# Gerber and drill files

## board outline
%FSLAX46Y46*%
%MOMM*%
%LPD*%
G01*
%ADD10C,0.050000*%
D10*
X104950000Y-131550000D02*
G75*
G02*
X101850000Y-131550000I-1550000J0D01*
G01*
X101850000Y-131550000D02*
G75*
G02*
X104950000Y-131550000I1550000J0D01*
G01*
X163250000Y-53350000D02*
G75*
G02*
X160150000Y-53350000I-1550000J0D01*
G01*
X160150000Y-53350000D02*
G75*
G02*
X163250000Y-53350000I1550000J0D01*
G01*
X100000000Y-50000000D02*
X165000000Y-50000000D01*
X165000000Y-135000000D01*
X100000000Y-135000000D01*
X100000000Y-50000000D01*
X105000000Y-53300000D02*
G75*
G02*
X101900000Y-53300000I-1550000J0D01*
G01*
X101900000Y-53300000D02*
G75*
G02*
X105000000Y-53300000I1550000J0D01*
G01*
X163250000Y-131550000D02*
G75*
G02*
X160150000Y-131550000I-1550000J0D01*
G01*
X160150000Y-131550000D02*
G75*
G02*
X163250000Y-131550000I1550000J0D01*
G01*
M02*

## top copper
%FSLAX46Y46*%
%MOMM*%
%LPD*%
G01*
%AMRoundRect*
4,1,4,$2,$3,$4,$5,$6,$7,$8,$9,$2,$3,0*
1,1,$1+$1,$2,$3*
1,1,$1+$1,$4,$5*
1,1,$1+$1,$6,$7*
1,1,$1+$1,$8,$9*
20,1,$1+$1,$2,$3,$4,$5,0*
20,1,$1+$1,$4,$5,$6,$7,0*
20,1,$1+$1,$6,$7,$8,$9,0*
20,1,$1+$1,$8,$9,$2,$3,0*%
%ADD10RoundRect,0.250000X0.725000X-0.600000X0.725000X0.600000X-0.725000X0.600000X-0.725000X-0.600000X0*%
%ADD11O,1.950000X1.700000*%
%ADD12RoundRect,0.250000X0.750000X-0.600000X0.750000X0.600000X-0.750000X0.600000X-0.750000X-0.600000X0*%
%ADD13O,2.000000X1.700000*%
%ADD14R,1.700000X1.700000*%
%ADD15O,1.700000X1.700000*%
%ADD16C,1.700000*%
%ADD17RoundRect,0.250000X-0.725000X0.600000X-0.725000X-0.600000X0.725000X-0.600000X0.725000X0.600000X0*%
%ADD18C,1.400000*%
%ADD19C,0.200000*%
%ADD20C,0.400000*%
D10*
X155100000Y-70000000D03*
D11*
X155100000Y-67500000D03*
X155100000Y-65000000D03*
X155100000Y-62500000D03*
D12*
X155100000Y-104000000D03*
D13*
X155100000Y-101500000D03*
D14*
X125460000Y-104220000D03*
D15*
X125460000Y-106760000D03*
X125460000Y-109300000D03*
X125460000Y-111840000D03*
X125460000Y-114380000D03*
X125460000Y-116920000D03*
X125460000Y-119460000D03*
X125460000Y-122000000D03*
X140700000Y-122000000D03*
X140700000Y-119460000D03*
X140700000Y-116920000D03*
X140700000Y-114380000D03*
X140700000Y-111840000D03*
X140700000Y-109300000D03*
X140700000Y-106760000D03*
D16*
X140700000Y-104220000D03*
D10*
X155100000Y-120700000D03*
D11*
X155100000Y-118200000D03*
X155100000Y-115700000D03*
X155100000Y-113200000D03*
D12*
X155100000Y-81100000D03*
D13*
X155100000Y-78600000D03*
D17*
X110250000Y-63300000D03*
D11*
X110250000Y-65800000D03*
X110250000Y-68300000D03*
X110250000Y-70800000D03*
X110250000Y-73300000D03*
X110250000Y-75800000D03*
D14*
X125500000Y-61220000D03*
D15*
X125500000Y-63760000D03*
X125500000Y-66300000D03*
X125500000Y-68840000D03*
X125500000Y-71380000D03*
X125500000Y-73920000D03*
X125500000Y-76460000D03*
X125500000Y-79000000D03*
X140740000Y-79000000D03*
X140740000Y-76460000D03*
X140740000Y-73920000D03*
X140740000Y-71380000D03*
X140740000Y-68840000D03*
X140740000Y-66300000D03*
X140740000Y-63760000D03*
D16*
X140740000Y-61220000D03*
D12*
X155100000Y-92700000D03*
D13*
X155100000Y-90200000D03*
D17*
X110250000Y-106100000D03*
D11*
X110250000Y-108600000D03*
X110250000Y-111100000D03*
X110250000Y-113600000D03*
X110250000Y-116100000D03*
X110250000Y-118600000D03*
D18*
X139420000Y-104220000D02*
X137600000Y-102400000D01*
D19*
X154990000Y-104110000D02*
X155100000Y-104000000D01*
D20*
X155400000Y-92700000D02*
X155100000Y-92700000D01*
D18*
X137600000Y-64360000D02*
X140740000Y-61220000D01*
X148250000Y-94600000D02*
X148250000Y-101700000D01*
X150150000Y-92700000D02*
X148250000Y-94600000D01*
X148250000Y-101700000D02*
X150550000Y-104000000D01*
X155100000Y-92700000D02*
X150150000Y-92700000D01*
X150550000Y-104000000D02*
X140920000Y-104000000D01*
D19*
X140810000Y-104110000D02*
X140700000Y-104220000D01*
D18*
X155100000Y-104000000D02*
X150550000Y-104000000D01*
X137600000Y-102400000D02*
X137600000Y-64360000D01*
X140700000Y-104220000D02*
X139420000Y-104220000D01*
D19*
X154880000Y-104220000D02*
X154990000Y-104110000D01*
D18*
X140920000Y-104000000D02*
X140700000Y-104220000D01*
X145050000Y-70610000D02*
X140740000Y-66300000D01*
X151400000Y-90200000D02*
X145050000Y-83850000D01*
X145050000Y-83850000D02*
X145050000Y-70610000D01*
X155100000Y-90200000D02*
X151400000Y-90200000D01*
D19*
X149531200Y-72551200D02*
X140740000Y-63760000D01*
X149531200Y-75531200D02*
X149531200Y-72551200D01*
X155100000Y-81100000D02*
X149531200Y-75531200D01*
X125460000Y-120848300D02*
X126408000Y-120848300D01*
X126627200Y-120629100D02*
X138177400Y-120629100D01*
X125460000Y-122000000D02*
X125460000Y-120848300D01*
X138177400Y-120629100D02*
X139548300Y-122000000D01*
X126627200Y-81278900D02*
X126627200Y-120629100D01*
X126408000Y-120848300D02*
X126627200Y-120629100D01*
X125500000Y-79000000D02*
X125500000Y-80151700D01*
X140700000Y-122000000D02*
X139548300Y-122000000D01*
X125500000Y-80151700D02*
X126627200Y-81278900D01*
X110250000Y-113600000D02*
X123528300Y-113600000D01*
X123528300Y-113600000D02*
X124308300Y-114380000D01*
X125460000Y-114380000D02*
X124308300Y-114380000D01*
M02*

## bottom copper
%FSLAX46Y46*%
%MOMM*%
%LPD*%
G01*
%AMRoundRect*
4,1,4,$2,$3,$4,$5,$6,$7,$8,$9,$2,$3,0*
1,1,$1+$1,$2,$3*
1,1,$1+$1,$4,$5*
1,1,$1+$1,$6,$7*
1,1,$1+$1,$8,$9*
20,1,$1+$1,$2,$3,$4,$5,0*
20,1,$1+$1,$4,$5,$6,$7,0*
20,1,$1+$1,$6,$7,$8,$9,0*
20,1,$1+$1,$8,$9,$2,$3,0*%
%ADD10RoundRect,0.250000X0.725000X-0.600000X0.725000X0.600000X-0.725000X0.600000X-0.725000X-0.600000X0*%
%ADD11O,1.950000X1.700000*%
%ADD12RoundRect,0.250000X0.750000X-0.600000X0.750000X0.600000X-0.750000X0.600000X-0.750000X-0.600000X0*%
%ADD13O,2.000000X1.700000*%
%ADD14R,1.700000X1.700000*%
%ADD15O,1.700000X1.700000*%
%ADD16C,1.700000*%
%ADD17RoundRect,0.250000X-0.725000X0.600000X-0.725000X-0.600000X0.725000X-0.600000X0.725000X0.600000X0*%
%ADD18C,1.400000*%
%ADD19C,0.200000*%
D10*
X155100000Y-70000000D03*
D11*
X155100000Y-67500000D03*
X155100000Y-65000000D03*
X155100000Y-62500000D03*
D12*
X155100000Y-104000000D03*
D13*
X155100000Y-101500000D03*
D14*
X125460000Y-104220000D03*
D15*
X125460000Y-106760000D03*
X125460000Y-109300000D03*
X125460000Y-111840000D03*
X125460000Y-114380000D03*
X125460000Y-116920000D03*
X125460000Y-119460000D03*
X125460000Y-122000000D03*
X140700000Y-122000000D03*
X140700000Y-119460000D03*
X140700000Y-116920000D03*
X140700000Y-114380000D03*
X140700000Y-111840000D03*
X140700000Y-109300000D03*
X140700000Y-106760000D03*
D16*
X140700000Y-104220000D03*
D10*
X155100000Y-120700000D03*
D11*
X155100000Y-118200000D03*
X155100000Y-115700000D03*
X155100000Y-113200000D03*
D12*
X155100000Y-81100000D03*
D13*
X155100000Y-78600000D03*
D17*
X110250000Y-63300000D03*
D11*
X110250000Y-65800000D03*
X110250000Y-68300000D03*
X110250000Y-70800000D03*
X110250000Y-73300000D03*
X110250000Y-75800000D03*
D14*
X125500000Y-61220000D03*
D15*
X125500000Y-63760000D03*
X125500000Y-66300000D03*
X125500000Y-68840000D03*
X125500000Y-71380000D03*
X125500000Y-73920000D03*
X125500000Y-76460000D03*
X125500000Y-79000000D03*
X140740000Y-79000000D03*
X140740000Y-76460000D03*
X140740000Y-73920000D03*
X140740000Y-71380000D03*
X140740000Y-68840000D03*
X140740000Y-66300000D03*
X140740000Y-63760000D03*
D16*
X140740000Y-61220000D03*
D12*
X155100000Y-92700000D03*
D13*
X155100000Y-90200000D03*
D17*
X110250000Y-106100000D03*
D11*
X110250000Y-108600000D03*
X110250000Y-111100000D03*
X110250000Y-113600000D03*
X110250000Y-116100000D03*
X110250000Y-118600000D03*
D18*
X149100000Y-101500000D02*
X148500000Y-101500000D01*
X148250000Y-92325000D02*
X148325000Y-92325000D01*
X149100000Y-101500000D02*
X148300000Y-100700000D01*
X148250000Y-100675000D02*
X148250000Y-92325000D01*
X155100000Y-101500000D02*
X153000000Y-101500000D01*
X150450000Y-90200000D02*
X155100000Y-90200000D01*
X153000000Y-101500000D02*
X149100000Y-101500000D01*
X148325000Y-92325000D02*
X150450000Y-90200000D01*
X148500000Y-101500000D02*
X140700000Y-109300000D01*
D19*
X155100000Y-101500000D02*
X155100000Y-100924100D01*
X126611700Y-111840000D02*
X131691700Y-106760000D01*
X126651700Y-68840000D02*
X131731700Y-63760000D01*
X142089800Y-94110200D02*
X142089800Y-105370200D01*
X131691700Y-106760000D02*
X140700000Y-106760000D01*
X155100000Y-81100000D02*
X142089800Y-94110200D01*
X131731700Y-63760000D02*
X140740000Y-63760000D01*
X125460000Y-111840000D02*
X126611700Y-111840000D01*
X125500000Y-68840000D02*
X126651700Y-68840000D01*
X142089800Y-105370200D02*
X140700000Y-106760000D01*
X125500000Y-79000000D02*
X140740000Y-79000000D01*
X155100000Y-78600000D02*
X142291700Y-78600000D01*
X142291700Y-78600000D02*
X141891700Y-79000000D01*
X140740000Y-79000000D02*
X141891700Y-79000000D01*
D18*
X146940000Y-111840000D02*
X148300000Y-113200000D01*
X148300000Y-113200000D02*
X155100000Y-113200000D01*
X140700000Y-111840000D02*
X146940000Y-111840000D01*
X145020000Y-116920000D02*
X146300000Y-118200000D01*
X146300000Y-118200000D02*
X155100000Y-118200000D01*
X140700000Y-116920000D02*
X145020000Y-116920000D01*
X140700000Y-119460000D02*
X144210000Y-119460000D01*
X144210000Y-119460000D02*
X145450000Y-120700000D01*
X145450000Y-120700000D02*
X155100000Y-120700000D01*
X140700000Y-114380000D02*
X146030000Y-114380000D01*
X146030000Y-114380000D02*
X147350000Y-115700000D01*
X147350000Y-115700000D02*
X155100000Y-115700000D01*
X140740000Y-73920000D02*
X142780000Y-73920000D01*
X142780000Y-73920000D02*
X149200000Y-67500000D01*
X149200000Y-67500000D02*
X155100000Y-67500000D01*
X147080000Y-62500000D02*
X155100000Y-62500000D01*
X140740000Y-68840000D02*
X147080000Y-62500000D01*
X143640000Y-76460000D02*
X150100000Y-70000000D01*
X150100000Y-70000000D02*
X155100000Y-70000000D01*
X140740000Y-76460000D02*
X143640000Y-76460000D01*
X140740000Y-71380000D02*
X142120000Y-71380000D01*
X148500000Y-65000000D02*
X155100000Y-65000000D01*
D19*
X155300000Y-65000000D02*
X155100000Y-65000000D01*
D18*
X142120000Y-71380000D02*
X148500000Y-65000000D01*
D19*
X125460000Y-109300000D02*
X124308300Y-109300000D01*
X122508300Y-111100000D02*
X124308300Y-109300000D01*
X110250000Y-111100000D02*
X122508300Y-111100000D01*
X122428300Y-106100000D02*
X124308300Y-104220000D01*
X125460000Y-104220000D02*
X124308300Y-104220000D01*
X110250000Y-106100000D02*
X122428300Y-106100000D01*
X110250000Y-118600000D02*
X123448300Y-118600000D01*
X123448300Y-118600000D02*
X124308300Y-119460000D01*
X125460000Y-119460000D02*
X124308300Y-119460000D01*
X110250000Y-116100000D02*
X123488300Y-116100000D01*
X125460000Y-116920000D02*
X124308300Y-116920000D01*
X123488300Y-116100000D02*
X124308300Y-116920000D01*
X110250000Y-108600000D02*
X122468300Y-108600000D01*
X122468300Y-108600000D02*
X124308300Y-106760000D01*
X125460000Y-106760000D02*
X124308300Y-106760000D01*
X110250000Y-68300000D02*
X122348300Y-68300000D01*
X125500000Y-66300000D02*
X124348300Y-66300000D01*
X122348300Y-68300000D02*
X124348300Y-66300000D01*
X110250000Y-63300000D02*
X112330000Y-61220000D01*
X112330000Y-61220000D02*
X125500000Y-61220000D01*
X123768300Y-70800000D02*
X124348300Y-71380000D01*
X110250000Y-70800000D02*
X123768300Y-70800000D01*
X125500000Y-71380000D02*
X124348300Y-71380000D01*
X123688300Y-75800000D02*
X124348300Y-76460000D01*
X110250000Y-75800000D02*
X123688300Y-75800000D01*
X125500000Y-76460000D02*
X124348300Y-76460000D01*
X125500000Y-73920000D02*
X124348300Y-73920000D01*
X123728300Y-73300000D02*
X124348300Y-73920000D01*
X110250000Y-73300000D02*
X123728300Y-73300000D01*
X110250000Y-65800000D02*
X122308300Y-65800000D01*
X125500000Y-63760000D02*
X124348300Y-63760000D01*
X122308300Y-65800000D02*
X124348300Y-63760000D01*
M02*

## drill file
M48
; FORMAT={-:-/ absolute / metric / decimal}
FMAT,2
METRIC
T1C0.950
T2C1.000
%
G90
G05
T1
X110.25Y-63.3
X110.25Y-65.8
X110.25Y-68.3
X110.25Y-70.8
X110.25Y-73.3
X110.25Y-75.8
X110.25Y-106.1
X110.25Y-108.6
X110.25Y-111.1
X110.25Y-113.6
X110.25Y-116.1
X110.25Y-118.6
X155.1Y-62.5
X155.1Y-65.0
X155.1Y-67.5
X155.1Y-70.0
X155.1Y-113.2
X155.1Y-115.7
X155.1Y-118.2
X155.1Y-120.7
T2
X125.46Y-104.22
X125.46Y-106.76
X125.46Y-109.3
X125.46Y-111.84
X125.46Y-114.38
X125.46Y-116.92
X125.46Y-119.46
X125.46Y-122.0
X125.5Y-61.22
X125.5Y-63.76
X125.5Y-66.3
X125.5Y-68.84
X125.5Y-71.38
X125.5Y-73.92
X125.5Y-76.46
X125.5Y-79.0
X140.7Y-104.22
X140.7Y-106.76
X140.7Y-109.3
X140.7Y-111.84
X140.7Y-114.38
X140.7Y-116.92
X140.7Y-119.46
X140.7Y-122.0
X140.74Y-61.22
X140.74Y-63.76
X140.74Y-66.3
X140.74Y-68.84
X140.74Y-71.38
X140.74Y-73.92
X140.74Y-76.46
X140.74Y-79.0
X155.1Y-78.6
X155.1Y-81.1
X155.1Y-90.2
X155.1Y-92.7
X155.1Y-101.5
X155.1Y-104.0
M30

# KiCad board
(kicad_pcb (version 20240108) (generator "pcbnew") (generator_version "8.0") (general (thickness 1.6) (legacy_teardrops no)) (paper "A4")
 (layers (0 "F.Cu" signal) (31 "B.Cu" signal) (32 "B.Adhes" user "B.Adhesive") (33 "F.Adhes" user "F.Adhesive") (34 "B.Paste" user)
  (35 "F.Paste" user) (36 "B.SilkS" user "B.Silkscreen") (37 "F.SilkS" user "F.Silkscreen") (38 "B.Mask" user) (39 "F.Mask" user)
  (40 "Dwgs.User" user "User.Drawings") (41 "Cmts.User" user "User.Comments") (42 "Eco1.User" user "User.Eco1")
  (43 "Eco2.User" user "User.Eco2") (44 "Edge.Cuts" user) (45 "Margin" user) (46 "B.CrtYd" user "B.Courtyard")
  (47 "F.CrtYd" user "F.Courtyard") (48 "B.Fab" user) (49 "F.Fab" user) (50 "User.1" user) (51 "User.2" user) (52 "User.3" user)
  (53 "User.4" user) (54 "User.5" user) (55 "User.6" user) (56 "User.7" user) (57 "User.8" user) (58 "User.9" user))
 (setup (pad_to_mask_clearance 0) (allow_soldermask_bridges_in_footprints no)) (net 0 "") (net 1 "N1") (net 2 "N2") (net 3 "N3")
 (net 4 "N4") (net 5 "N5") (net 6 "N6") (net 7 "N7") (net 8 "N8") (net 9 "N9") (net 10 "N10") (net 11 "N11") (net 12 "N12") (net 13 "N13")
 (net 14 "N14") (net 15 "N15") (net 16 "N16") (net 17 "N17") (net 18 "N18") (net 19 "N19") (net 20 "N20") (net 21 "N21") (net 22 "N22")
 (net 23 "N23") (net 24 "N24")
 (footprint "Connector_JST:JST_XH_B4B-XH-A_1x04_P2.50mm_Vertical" (layer "F.Cu") (at 155.1 70 90)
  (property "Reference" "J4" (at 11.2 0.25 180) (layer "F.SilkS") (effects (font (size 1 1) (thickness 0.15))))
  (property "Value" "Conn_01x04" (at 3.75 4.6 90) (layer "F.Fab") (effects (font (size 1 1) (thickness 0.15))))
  (pad "1" thru_hole roundrect (at 0 0 90) (size 1.7 1.95) (drill 0.95) (layers "*.Cu" "*.Mask") (remove_unused_layers no)
   (roundrect_rratio 0.147059) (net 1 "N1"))
  (pad "2" thru_hole oval (at 2.5 0 90) (size 1.7 1.95) (drill 0.95) (layers "*.Cu" "*.Mask") (remove_unused_layers no) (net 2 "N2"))
  (pad "3" thru_hole oval (at 5 0 90) (size 1.7 1.95) (drill 0.95) (layers "*.Cu" "*.Mask") (remove_unused_layers no) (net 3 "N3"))
  (pad "4" thru_hole oval (at 7.5 0 90) (size 1.7 1.95) (drill 0.95) (layers "*.Cu" "*.Mask") (remove_unused_layers no) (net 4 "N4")))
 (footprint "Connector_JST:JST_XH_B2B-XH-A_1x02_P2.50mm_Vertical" (layer "F.Cu") (at 155.1 104 90)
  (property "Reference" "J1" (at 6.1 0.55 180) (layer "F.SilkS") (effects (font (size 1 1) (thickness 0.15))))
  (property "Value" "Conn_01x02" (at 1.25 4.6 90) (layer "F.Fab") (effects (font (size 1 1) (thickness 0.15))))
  (pad "1" thru_hole roundrect (at 0 0 90) (size 1.7 2) (drill 1) (layers "*.Cu" "*.Mask") (remove_unused_layers no)
   (roundrect_rratio 0.147059) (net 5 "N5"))
  (pad "2" thru_hole oval (at 2.5 0 90) (size 1.7 2) (drill 1) (layers "*.Cu" "*.Mask") (remove_unused_layers no) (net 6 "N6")))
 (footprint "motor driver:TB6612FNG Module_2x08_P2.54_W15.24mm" (layer "F.Cu") (at 125.46 104.22)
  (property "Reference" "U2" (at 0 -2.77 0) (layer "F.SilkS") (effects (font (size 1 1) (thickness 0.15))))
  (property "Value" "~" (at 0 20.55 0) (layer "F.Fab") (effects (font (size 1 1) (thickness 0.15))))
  (pad "1" thru_hole rect (at 0 0) (size 1.7 1.7) (drill 1) (layers "*.Cu" "*.Mask") (remove_unused_layers no) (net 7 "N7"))
  (pad "2" thru_hole oval (at 0 2.54) (size 1.7 1.7) (drill 1) (layers "*.Cu" "*.Mask") (remove_unused_layers no) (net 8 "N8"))
  (pad "3" thru_hole oval (at 0 5.08) (size 1.7 1.7) (drill 1) (layers "*.Cu" "*.Mask") (remove_unused_layers no) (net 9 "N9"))
  (pad "4" thru_hole oval (at 0 7.62) (size 1.7 1.7) (drill 1) (layers "*.Cu" "*.Mask") (remove_unused_layers no) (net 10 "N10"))
  (pad "5" thru_hole oval (at 0 10.16) (size 1.7 1.7) (drill 1) (layers "*.Cu" "*.Mask") (remove_unused_layers no) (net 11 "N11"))
  (pad "6" thru_hole oval (at 0 12.7) (size 1.7 1.7) (drill 1) (layers "*.Cu" "*.Mask") (remove_unused_layers no) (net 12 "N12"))
  (pad "7" thru_hole oval (at 0 15.24) (size 1.7 1.7) (drill 1) (layers "*.Cu" "*.Mask") (remove_unused_layers no) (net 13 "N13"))
  (pad "8" thru_hole oval (at 0 17.78) (size 1.7 1.7) (drill 1) (layers "*.Cu" "*.Mask") (remove_unused_layers no) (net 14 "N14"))
  (pad "9" thru_hole oval (at 15.24 17.78) (size 1.7 1.7) (drill 1) (layers "*.Cu" "*.Mask") (remove_unused_layers no) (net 14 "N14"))
  (pad "10" thru_hole oval (at 15.24 15.24) (size 1.7 1.7) (drill 1) (layers "*.Cu" "*.Mask") (remove_unused_layers no) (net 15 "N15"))
  (pad "11" thru_hole oval (at 15.24 12.7) (size 1.7 1.7) (drill 1) (layers "*.Cu" "*.Mask") (remove_unused_layers no) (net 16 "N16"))
  (pad "12" thru_hole oval (at 15.24 10.16) (size 1.7 1.7) (drill 1) (layers "*.Cu" "*.Mask") (remove_unused_layers no) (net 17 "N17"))
  (pad "13" thru_hole oval (at 15.24 7.62) (size 1.7 1.7) (drill 1) (layers "*.Cu" "*.Mask") (remove_unused_layers no) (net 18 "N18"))
  (pad "14" thru_hole oval (at 15.24 5.08) (size 1.7 1.7) (drill 1) (layers "*.Cu" "*.Mask") (remove_unused_layers no) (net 6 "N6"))
  (pad "15" thru_hole oval (at 15.24 2.54) (size 1.7 1.7) (drill 1) (layers "*.Cu" "*.Mask") (remove_unused_layers no) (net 10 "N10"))
  (pad "16" thru_hole circle (at 15.24 0) (size 1.7 1.7) (drill 1) (layers "*.Cu" "*.Mask") (remove_unused_layers no) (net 5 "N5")))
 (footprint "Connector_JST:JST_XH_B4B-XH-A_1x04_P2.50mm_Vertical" (layer "F.Cu") (at 155.1 120.7 90)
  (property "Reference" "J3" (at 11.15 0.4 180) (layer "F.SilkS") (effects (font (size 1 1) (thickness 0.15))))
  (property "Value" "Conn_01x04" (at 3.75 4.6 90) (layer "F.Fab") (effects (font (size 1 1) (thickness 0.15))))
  (pad "1" thru_hole roundrect (at 0 0 90) (size 1.7 1.95) (drill 0.95) (layers "*.Cu" "*.Mask") (remove_unused_layers no)
   (roundrect_rratio 0.147059) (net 15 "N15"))
  (pad "2" thru_hole oval (at 2.5 0 90) (size 1.7 1.95) (drill 0.95) (layers "*.Cu" "*.Mask") (remove_unused_layers no) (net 16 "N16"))
  (pad "3" thru_hole oval (at 5 0 90) (size 1.7 1.95) (drill 0.95) (layers "*.Cu" "*.Mask") (remove_unused_layers no) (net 17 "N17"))
  (pad "4" thru_hole oval (at 7.5 0 90) (size 1.7 1.95) (drill 0.95) (layers "*.Cu" "*.Mask") (remove_unused_layers no) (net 18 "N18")))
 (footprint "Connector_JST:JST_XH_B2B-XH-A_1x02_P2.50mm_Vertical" (layer "F.Cu") (at 155.1 81.1 90)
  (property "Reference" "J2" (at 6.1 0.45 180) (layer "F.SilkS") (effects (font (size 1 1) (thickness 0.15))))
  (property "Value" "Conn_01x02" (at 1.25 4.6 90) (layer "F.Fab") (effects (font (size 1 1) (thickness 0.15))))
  (pad "1" thru_hole roundrect (at 0 0 90) (size 1.7 2) (drill 1) (layers "*.Cu" "*.Mask") (remove_unused_layers no)
   (roundrect_rratio 0.147059) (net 10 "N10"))
  (pad "2" thru_hole oval (at 2.5 0 90) (size 1.7 2) (drill 1) (layers "*.Cu" "*.Mask") (remove_unused_layers no) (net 14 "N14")))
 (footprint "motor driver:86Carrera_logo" (layer "F.Cu") (at 111.2 128.35)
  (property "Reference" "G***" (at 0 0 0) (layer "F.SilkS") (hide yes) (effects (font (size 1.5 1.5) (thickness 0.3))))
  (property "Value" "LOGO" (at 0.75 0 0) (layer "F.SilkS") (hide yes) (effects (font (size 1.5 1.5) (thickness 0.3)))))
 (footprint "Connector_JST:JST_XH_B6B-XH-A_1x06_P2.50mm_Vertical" (layer "F.Cu") (at 110.25 63.3 -90)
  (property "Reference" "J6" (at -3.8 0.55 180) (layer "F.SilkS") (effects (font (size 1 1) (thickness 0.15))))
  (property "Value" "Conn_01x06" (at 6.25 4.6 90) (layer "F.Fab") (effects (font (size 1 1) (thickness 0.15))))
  (pad "1" thru_hole roundrect (at 0 0 270) (size 1.7 1.95) (drill 0.95) (layers "*.Cu" "*.Mask") (remove_unused_layers no)
   (roundrect_rratio 0.147059) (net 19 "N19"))
  (pad "2" thru_hole oval (at 2.5 0 270) (size 1.7 1.95) (drill 0.95) (layers "*.Cu" "*.Mask") (remove_unused_layers no) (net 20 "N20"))
  (pad "3" thru_hole oval (at 5 0 270) (size 1.7 1.95) (drill 0.95) (layers "*.Cu" "*.Mask") (remove_unused_layers no) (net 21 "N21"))
  (pad "4" thru_hole oval (at 7.5 0 270) (size 1.7 1.95) (drill 0.95) (layers "*.Cu" "*.Mask") (remove_unused_layers no) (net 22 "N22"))
  (pad "5" thru_hole oval (at 10 0 270) (size 1.7 1.95) (drill 0.95) (layers "*.Cu" "*.Mask") (remove_unused_layers no) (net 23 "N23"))
  (pad "6" thru_hole oval (at 12.5 0 270) (size 1.7 1.95) (drill 0.95) (layers "*.Cu" "*.Mask") (remove_unused_layers no) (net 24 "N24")))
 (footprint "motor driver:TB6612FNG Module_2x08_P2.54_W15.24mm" (layer "F.Cu") (at 125.5 61.22)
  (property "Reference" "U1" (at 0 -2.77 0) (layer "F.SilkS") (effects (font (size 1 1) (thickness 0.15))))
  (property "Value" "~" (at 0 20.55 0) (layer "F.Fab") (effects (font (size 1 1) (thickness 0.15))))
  (pad "1" thru_hole rect (at 0 0) (size 1.7 1.7) (drill 1) (layers "*.Cu" "*.Mask") (remove_unused_layers no) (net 19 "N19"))
  (pad "2" thru_hole oval (at 0 2.54) (size 1.7 1.7) (drill 1) (layers "*.Cu" "*.Mask") (remove_unused_layers no) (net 20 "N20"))
  (pad "3" thru_hole oval (at 0 5.08) (size 1.7 1.7) (drill 1) (layers "*.Cu" "*.Mask") (remove_unused_layers no) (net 21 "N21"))
  (pad "4" thru_hole oval (at 0 7.62) (size 1.7 1.7) (drill 1) (layers "*.Cu" "*.Mask") (remove_unused_layers no) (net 10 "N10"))
  (pad "5" thru_hole oval (at 0 10.16) (size 1.7 1.7) (drill 1) (layers "*.Cu" "*.Mask") (remove_unused_layers no) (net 22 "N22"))
  (pad "6" thru_hole oval (at 0 12.7) (size 1.7 1.7) (drill 1) (layers "*.Cu" "*.Mask") (remove_unused_layers no) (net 23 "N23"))
  (pad "7" thru_hole oval (at 0 15.24) (size 1.7 1.7) (drill 1) (layers "*.Cu" "*.Mask") (remove_unused_layers no) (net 24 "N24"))
  (pad "8" thru_hole oval (at 0 17.78) (size 1.7 1.7) (drill 1) (layers "*.Cu" "*.Mask") (remove_unused_layers no) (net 14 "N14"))
  (pad "9" thru_hole oval (at 15.24 17.78) (size 1.7 1.7) (drill 1) (layers "*.Cu" "*.Mask") (remove_unused_layers no) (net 14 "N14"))
  (pad "10" thru_hole oval (at 15.24 15.24) (size 1.7 1.7) (drill 1) (layers "*.Cu" "*.Mask") (remove_unused_layers no) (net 1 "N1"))
  (pad "11" thru_hole oval (at 15.24 12.7) (size 1.7 1.7) (drill 1) (layers "*.Cu" "*.Mask") (remove_unused_layers no) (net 2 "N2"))
  (pad "12" thru_hole oval (at 15.24 10.16) (size 1.7 1.7) (drill 1) (layers "*.Cu" "*.Mask") (remove_unused_layers no) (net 3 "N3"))
  (pad "13" thru_hole oval (at 15.24 7.62) (size 1.7 1.7) (drill 1) (layers "*.Cu" "*.Mask") (remove_unused_layers no) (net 4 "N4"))
  (pad "14" thru_hole oval (at 15.24 5.08) (size 1.7 1.7) (drill 1) (layers "*.Cu" "*.Mask") (remove_unused_layers no) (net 6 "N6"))
  (pad "15" thru_hole oval (at 15.24 2.54) (size 1.7 1.7) (drill 1) (layers "*.Cu" "*.Mask") (remove_unused_layers no) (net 10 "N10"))
  (pad "16" thru_hole circle (at 15.24 0) (size 1.7 1.7) (drill 1) (layers "*.Cu" "*.Mask") (remove_unused_layers no) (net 5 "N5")))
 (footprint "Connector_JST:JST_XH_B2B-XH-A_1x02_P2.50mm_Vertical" (layer "F.Cu") (at 155.1 92.7 90)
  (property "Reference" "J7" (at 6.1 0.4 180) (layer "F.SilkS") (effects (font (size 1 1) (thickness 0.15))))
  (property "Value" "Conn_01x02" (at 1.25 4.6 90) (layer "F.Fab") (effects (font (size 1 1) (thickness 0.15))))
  (pad "1" thru_hole roundrect (at 0 0 90) (size 1.7 2) (drill 1) (layers "*.Cu" "*.Mask") (remove_unused_layers no)
   (roundrect_rratio 0.147059) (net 5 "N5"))
  (pad "2" thru_hole oval (at 2.5 0 90) (size 1.7 2) (drill 1) (layers "*.Cu" "*.Mask") (remove_unused_layers no) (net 6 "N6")))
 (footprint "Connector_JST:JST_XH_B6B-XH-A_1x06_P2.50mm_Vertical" (layer "F.Cu") (at 110.25 106.1 -90)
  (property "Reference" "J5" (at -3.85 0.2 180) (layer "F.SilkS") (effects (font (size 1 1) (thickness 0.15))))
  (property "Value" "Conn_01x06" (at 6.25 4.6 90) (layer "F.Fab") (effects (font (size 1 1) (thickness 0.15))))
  (pad "1" thru_hole roundrect (at 0 0 270) (size 1.7 1.95) (drill 0.95) (layers "*.Cu" "*.Mask") (remove_unused_layers no)
   (roundrect_rratio 0.147059) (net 7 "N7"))
  (pad "2" thru_hole oval (at 2.5 0 270) (size 1.7 1.95) (drill 0.95) (layers "*.Cu" "*.Mask") (remove_unused_layers no) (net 8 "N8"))
  (pad "3" thru_hole oval (at 5 0 270) (size 1.7 1.95) (drill 0.95) (layers "*.Cu" "*.Mask") (remove_unused_layers no) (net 9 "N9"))
  (pad "4" thru_hole oval (at 7.5 0 270) (size 1.7 1.95) (drill 0.95) (layers "*.Cu" "*.Mask") (remove_unused_layers no) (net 11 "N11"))
  (pad "5" thru_hole oval (at 10 0 270) (size 1.7 1.95) (drill 0.95) (layers "*.Cu" "*.Mask") (remove_unused_layers no) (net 12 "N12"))
  (pad "6" thru_hole oval (at 12.5 0 270) (size 1.7 1.95) (drill 0.95) (layers "*.Cu" "*.Mask") (remove_unused_layers no) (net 13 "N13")))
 (gr_circle (center 103.4 131.55) (end 104.95 131.55) (stroke (width 0.05) (type default)) (fill none) (layer "Edge.Cuts"))
 (gr_circle (center 161.7 53.35) (end 163.25 53.35) (stroke (width 0.05) (type default)) (fill none) (layer "Edge.Cuts"))
 (gr_rect (start 100 50) (end 165 135) (locked yes) (stroke (width 0.05) (type default)) (fill none) (layer "Edge.Cuts"))
 (gr_circle (center 103.45 53.3) (end 105 53.3) (stroke (width 0.05) (type default)) (fill none) (layer "Edge.Cuts"))
 (gr_circle (center 161.7 131.55) (end 163.25 131.55) (stroke (width 0.05) (type default)) (fill none) (layer "Edge.Cuts"))
 (segment (start 139.42 104.22) (end 137.6 102.4) (width 1.4) (layer "F.Cu") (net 5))
 (segment (start 154.99 104.11) (end 155.1 104) (width 0.2) (layer "F.Cu") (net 5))
 (segment (start 155.4 92.7) (end 155.1 92.7) (width 0.4) (layer "F.Cu") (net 5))
 (segment (start 137.6 64.36) (end 140.74 61.22) (width 1.4) (layer "F.Cu") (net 5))
 (segment (start 148.25 94.6) (end 148.25 101.7) (width 1.4) (layer "F.Cu") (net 5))
 (segment (start 150.15 92.7) (end 148.25 94.6) (width 1.4) (layer "F.Cu") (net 5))
 (segment (start 148.25 101.7) (end 150.55 104) (width 1.4) (layer "F.Cu") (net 5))
 (segment (start 155.1 92.7) (end 150.15 92.7) (width 1.4) (layer "F.Cu") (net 5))
 (segment (start 150.55 104) (end 140.92 104) (width 1.4) (layer "F.Cu") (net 5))
 (segment (start 140.81 104.11) (end 140.7 104.22) (width 0.2) (layer "F.Cu") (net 5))
 (segment (start 155.1 104) (end 150.55 104) (width 1.4) (layer "F.Cu") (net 5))
 (segment (start 137.6 102.4) (end 137.6 64.36) (width 1.4) (layer "F.Cu") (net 5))
 (segment (start 140.7 104.22) (end 139.42 104.22) (width 1.4) (layer "F.Cu") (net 5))
 (segment (start 154.88 104.22) (end 154.99 104.11) (width 0.2) (layer "F.Cu") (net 5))
 (segment (start 140.92 104) (end 140.7 104.22) (width 1.4) (layer "F.Cu") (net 5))
 (segment (start 145.05 70.61) (end 140.74 66.3) (width 1.4) (layer "F.Cu") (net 6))
 (segment (start 151.4 90.2) (end 145.05 83.85) (width 1.4) (layer "F.Cu") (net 6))
 (segment (start 145.05 83.85) (end 145.05 70.61) (width 1.4) (layer "F.Cu") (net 6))
 (segment (start 155.1 90.2) (end 151.4 90.2) (width 1.4) (layer "F.Cu") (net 6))
 (segment (start 149.1 101.5) (end 148.5 101.5) (width 1.4) (layer "B.Cu") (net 6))
 (segment (start 148.25 92.325) (end 148.325 92.325) (width 1.4) (layer "B.Cu") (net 6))
 (segment (start 149.1 101.5) (end 148.3 100.7) (width 1.4) (layer "B.Cu") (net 6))
 (segment (start 148.25 100.675) (end 148.25 92.325) (width 1.4) (layer "B.Cu") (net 6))
 (segment (start 155.1 101.5) (end 153 101.5) (width 1.4) (layer "B.Cu") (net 6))
 (segment (start 150.45 90.2) (end 155.1 90.2) (width 1.4) (layer "B.Cu") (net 6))
 (segment (start 153 101.5) (end 149.1 101.5) (width 1.4) (layer "B.Cu") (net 6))
 (segment (start 148.325 92.325) (end 150.45 90.2) (width 1.4) (layer "B.Cu") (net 6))
 (segment (start 148.5 101.5) (end 140.7 109.3) (width 1.4) (layer "B.Cu") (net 6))
 (segment (start 155.1 101.5) (end 155.1 100.9241) (width 0.2) (layer "B.Cu") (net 6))
 (segment (start 149.5312 72.5512) (end 140.74 63.76) (width 0.2) (layer "F.Cu") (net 10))
 (segment (start 149.5312 75.5312) (end 149.5312 72.5512) (width 0.2) (layer "F.Cu") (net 10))
 (segment (start 155.1 81.1) (end 149.5312 75.5312) (width 0.2) (layer "F.Cu") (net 10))
 (segment (start 126.6117 111.84) (end 131.6917 106.76) (width 0.2) (layer "B.Cu") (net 10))
 (segment (start 126.6517 68.84) (end 131.7317 63.76) (width 0.2) (layer "B.Cu") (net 10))
 (segment (start 142.0898 94.1102) (end 142.0898 105.3702) (width 0.2) (layer "B.Cu") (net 10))
 (segment (start 131.6917 106.76) (end 140.7 106.76) (width 0.2) (layer "B.Cu") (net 10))
 (segment (start 155.1 81.1) (end 142.0898 94.1102) (width 0.2) (layer "B.Cu") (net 10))
 (segment (start 131.7317 63.76) (end 140.74 63.76) (width 0.2) (layer "B.Cu") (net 10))
 (segment (start 125.46 111.84) (end 126.6117 111.84) (width 0.2) (layer "B.Cu") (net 10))
 (segment (start 125.5 68.84) (end 126.6517 68.84) (width 0.2) (layer "B.Cu") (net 10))
 (segment (start 142.0898 105.3702) (end 140.7 106.76) (width 0.2) (layer "B.Cu") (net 10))
 (segment (start 125.46 120.8483) (end 126.408 120.8483) (width 0.2) (layer "F.Cu") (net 14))
 (segment (start 126.6272 120.6291) (end 138.1774 120.6291) (width 0.2) (layer "F.Cu") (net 14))
 (segment (start 125.46 122) (end 125.46 120.8483) (width 0.2) (layer "F.Cu") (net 14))
 (segment (start 138.1774 120.6291) (end 139.5483 122) (width 0.2) (layer "F.Cu") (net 14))
 (segment (start 126.6272 81.2789) (end 126.6272 120.6291) (width 0.2) (layer "F.Cu") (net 14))
 (segment (start 126.408 120.8483) (end 126.6272 120.6291) (width 0.2) (layer "F.Cu") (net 14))
 (segment (start 125.5 79) (end 125.5 80.1517) (width 0.2) (layer "F.Cu") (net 14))
 (segment (start 140.7 122) (end 139.5483 122) (width 0.2) (layer "F.Cu") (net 14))
 (segment (start 125.5 80.1517) (end 126.6272 81.2789) (width 0.2) (layer "F.Cu") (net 14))
 (segment (start 125.5 79) (end 140.74 79) (width 0.2) (layer "B.Cu") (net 14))
 (segment (start 155.1 78.6) (end 142.2917 78.6) (width 0.2) (layer "B.Cu") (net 14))
 (segment (start 142.2917 78.6) (end 141.8917 79) (width 0.2) (layer "B.Cu") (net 14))
 (segment (start 140.74 79) (end 141.8917 79) (width 0.2) (layer "B.Cu") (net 14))
 (segment (start 146.94 111.84) (end 148.3 113.2) (width 1.4) (layer "B.Cu") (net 18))
 (segment (start 148.3 113.2) (end 155.1 113.2) (width 1.4) (layer "B.Cu") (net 18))
 (segment (start 140.7 111.84) (end 146.94 111.84) (width 1.4) (layer "B.Cu") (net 18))
 (segment (start 145.02 116.92) (end 146.3 118.2) (width 1.4) (layer "B.Cu") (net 16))
 (segment (start 146.3 118.2) (end 155.1 118.2) (width 1.4) (layer "B.Cu") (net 16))
 (segment (start 140.7 116.92) (end 145.02 116.92) (width 1.4) (layer "B.Cu") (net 16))
 (segment (start 140.7 119.46) (end 144.21 119.46) (width 1.4) (layer "B.Cu") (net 15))
 (segment (start 144.21 119.46) (end 145.45 120.7) (width 1.4) (layer "B.Cu") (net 15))
 (segment (start 145.45 120.7) (end 155.1 120.7) (width 1.4) (layer "B.Cu") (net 15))
 (segment (start 140.7 114.38) (end 146.03 114.38) (width 1.4) (layer "B.Cu") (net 17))
 (segment (start 146.03 114.38) (end 147.35 115.7) (width 1.4) (layer "B.Cu") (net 17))
 (segment (start 147.35 115.7) (end 155.1 115.7) (width 1.4) (layer "B.Cu") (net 17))
 (segment (start 140.74 73.92) (end 142.78 73.92) (width 1.4) (layer "B.Cu") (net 2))
 (segment (start 142.78 73.92) (end 149.2 67.5) (width 1.4) (layer "B.Cu") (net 2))
 (segment (start 149.2 67.5) (end 155.1 67.5) (width 1.4) (layer "B.Cu") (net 2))
 (segment (start 147.08 62.5) (end 155.1 62.5) (width 1.4) (layer "B.Cu") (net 4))
 (segment (start 140.74 68.84) (end 147.08 62.5) (width 1.4) (layer "B.Cu") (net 4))
 (segment (start 143.64 76.46) (end 150.1 70) (width 1.4) (layer "B.Cu") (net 1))
 (segment (start 150.1 70) (end 155.1 70) (width 1.4) (layer "B.Cu") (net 1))
 (segment (start 140.74 76.46) (end 143.64 76.46) (width 1.4) (layer "B.Cu") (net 1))
 (segment (start 140.74 71.38) (end 142.12 71.38) (width 1.4) (layer "B.Cu") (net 3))
 (segment (start 148.5 65) (end 155.1 65) (width 1.4) (layer "B.Cu") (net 3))
 (segment (start 155.3 65) (end 155.1 65) (width 0.2) (layer "B.Cu") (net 3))
 (segment (start 142.12 71.38) (end 148.5 65) (width 1.4) (layer "B.Cu") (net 3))
 (segment (start 125.46 109.3) (end 124.3083 109.3) (width 0.2) (layer "B.Cu") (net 9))
 (segment (start 122.5083 111.1) (end 124.3083 109.3) (width 0.2) (layer "B.Cu") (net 9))
 (segment (start 110.25 111.1) (end 122.5083 111.1) (width 0.2) (layer "B.Cu") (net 9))
 (segment (start 122.4283 106.1) (end 124.3083 104.22) (width 0.2) (layer "B.Cu") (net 7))
 (segment (start 125.46 104.22) (end 124.3083 104.22) (width 0.2) (layer "B.Cu") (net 7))
 (segment (start 110.25 106.1) (end 122.4283 106.1) (width 0.2) (layer "B.Cu") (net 7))
 (segment (start 110.25 118.6) (end 123.4483 118.6) (width 0.2) (layer "B.Cu") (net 13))
 (segment (start 123.4483 118.6) (end 124.3083 119.46) (width 0.2) (layer "B.Cu") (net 13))
 (segment (start 125.46 119.46) (end 124.3083 119.46) (width 0.2) (layer "B.Cu") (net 13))
 (segment (start 110.25 116.1) (end 123.4883 116.1) (width 0.2) (layer "B.Cu") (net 12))
 (segment (start 125.46 116.92) (end 124.3083 116.92) (width 0.2) (layer "B.Cu") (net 12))
 (segment (start 123.4883 116.1) (end 124.3083 116.92) (width 0.2) (layer "B.Cu") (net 12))
 (segment (start 110.25 113.6) (end 123.5283 113.6) (width 0.2) (layer "F.Cu") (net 11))
 (segment (start 123.5283 113.6) (end 124.3083 114.38) (width 0.2) (layer "F.Cu") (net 11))
 (segment (start 125.46 114.38) (end 124.3083 114.38) (width 0.2) (layer "F.Cu") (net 11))
 (segment (start 110.25 108.6) (end 122.4683 108.6) (width 0.2) (layer "B.Cu") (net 8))
 (segment (start 122.4683 108.6) (end 124.3083 106.76) (width 0.2) (layer "B.Cu") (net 8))
 (segment (start 125.46 106.76) (end 124.3083 106.76) (width 0.2) (layer "B.Cu") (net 8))
 (segment (start 110.25 68.3) (end 122.3483 68.3) (width 0.2) (layer "B.Cu") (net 21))
 (segment (start 125.5 66.3) (end 124.3483 66.3) (width 0.2) (layer "B.Cu") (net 21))
 (segment (start 122.3483 68.3) (end 124.3483 66.3) (width 0.2) (layer "B.Cu") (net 21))
 (segment (start 110.25 63.3) (end 112.33 61.22) (width 0.2) (layer "B.Cu") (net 19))
 (segment (start 112.33 61.22) (end 125.5 61.22) (width 0.2) (layer "B.Cu") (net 19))
 (segment (start 123.7683 70.8) (end 124.3483 71.38) (width 0.2) (layer "B.Cu") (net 22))
 (segment (start 110.25 70.8) (end 123.7683 70.8) (width 0.2) (layer "B.Cu") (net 22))
 (segment (start 125.5 71.38) (end 124.3483 71.38) (width 0.2) (layer "B.Cu") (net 22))
 (segment (start 123.6883 75.8) (end 124.3483 76.46) (width 0.2) (layer "B.Cu") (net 24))
 (segment (start 110.25 75.8) (end 123.6883 75.8) (width 0.2) (layer "B.Cu") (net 24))
 (segment (start 125.5 76.46) (end 124.3483 76.46) (width 0.2) (layer "B.Cu") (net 24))
 (segment (start 125.5 73.92) (end 124.3483 73.92) (width 0.2) (layer "B.Cu") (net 23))
 (segment (start 123.7283 73.3) (end 124.3483 73.92) (width 0.2) (layer "B.Cu") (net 23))
 (segment (start 110.25 73.3) (end 123.7283 73.3) (width 0.2) (layer "B.Cu") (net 23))
 (segment (start 110.25 65.8) (end 122.3083 65.8) (width 0.2) (layer "B.Cu") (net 20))
 (segment (start 125.5 63.76) (end 124.3483 63.76) (width 0.2) (layer "B.Cu") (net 20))
 (segment (start 122.3083 65.8) (end 124.3483 63.76) (width 0.2) (layer "B.Cu") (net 20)))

